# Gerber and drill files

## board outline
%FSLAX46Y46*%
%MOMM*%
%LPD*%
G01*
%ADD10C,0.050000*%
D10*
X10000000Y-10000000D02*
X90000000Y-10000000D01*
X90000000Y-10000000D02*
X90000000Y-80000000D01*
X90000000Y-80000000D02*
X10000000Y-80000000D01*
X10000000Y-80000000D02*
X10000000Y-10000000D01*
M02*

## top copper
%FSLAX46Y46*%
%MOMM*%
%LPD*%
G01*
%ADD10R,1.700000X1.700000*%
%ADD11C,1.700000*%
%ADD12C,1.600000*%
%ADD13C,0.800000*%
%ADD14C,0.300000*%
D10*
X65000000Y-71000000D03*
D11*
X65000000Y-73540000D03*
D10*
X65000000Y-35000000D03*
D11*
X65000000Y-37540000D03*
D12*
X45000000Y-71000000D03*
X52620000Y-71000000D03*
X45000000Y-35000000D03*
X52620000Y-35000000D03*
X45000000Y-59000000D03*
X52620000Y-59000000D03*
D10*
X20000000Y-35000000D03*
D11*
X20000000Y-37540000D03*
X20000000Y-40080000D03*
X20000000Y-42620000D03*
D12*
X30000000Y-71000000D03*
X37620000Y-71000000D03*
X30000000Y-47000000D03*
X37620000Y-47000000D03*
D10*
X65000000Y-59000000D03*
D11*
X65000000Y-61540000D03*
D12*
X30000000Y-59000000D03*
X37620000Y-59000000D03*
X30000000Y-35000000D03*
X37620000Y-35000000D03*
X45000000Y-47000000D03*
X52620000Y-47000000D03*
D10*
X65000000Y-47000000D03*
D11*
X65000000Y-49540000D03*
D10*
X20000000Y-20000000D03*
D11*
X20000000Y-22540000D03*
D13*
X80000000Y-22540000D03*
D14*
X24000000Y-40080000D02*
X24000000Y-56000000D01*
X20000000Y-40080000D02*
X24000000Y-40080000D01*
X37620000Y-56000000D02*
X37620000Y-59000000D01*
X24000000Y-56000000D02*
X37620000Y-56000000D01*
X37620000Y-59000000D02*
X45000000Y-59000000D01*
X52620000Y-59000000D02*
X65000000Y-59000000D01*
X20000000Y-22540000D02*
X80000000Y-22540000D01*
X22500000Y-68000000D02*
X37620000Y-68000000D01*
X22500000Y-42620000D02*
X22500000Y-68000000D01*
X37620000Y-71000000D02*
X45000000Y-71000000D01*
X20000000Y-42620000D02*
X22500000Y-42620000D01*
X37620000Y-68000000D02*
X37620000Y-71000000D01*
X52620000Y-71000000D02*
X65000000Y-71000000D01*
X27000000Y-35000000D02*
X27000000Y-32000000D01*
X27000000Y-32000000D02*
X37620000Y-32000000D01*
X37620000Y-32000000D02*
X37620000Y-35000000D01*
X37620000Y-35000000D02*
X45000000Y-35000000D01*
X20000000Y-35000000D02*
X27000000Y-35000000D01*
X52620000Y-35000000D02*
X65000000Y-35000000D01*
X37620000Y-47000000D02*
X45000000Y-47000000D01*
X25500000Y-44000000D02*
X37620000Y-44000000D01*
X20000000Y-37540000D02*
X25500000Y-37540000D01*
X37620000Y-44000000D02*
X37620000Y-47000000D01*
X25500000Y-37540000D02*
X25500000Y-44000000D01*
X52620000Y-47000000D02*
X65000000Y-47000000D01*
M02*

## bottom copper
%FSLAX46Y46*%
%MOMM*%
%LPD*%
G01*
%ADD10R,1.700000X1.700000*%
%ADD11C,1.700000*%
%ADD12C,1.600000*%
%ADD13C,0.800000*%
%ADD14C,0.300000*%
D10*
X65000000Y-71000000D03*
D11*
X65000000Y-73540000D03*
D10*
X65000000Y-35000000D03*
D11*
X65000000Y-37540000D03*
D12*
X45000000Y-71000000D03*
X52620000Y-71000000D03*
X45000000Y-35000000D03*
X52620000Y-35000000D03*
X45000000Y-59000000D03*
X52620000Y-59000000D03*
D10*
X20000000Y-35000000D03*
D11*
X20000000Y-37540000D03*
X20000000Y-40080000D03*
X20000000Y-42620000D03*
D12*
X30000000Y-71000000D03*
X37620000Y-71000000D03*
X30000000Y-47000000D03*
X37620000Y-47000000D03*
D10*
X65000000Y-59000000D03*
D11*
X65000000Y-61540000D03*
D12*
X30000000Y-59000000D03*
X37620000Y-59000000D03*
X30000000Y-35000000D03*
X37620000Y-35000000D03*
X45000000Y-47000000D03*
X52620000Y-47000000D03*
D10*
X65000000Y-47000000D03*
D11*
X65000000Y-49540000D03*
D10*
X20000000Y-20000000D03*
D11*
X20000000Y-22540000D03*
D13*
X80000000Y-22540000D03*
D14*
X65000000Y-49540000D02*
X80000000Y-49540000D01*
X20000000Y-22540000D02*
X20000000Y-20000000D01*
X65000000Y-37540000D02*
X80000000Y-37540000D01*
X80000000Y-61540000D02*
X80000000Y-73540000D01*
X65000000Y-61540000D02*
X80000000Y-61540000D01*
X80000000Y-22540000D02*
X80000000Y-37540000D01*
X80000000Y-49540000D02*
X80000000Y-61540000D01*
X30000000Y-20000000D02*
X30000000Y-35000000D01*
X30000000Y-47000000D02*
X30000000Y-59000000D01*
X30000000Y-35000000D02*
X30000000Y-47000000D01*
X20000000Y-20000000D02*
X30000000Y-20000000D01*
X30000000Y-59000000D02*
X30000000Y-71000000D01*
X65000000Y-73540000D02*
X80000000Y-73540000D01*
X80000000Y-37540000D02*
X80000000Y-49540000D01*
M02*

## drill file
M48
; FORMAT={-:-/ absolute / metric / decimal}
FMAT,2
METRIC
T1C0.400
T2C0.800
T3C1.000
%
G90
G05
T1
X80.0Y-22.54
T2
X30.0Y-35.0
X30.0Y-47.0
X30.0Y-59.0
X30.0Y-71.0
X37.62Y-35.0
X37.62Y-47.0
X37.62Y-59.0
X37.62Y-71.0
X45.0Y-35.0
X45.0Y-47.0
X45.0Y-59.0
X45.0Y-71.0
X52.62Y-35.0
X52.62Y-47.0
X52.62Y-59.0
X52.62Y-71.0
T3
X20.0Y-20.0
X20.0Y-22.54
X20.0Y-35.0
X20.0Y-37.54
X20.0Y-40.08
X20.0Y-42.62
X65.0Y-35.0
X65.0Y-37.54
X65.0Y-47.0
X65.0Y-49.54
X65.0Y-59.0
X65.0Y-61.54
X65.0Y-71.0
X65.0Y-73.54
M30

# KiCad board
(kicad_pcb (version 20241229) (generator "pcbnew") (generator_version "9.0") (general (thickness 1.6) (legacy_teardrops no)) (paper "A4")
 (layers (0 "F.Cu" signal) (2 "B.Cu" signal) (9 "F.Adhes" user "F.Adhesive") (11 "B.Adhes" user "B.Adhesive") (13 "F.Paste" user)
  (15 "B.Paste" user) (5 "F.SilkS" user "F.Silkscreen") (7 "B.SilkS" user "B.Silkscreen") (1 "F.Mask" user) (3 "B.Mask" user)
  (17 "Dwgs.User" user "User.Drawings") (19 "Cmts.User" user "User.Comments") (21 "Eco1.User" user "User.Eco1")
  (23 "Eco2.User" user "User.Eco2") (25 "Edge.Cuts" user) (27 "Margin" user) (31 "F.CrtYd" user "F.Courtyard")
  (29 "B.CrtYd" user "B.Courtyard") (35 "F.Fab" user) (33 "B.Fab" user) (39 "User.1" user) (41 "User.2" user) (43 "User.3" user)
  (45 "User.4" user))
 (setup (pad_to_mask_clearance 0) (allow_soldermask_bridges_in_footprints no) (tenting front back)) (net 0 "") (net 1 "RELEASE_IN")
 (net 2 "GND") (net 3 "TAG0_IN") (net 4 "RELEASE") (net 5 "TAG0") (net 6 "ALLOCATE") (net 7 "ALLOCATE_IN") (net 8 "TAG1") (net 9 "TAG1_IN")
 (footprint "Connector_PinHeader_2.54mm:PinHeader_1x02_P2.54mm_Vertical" (layer "F.Cu") (at 65 71)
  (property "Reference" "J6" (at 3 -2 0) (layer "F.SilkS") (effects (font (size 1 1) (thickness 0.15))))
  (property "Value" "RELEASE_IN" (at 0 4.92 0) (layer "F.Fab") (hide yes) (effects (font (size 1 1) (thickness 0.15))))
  (pad "1" thru_hole rect (at 0 0) (size 1.7 1.7) (drill 1) (layers "*.Cu" "*.Mask") (remove_unused_layers no) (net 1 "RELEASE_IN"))
  (pad "2" thru_hole circle (at 0 2.54) (size 1.7 1.7) (drill 1) (layers "*.Cu" "*.Mask") (remove_unused_layers no) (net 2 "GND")))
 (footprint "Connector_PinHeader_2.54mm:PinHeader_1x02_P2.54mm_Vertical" (layer "F.Cu") (at 65 35)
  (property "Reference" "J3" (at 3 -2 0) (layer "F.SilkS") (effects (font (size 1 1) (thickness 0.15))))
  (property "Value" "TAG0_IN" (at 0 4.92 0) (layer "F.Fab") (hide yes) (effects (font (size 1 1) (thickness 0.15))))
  (pad "1" thru_hole rect (at 0 0) (size 1.7 1.7) (drill 1) (layers "*.Cu" "*.Mask") (remove_unused_layers no) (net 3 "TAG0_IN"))
  (pad "2" thru_hole circle (at 0 2.54) (size 1.7 1.7) (drill 1) (layers "*.Cu" "*.Mask") (remove_unused_layers no) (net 2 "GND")))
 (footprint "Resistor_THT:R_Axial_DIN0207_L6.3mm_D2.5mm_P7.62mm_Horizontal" (layer "F.Cu") (at 45 71)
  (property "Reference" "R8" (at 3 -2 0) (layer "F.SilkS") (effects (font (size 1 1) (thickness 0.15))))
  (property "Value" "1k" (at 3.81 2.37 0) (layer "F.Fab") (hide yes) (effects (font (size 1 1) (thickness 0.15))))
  (pad "1" thru_hole circle (at 0 0) (size 1.6 1.6) (drill 0.8) (layers "*.Cu" "*.Mask") (remove_unused_layers no) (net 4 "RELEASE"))
  (pad "2" thru_hole circle (at 7.62 0) (size 1.6 1.6) (drill 0.8) (layers "*.Cu" "*.Mask") (remove_unused_layers no) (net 1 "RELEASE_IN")))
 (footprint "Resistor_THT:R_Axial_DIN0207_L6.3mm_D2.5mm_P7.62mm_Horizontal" (layer "F.Cu") (at 45 35)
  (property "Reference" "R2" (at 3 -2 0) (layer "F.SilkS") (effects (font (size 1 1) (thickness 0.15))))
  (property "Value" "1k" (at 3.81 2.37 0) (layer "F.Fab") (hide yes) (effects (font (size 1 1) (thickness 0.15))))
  (pad "1" thru_hole circle (at 0 0) (size 1.6 1.6) (drill 0.8) (layers "*.Cu" "*.Mask") (remove_unused_layers no) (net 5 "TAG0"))
  (pad "2" thru_hole circle (at 7.62 0) (size 1.6 1.6) (drill 0.8) (layers "*.Cu" "*.Mask") (remove_unused_layers no) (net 3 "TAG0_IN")))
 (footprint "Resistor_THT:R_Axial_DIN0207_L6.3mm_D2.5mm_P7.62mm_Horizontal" (layer "F.Cu") (at 45 59)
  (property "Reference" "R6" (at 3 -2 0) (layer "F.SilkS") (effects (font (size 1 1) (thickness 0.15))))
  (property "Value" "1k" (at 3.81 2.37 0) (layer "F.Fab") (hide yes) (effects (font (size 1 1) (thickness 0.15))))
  (pad "1" thru_hole circle (at 0 0) (size 1.6 1.6) (drill 0.8) (layers "*.Cu" "*.Mask") (remove_unused_layers no) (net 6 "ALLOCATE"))
  (pad "2" thru_hole circle (at 7.62 0) (size 1.6 1.6) (drill 0.8) (layers "*.Cu" "*.Mask") (remove_unused_layers no) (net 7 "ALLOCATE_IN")))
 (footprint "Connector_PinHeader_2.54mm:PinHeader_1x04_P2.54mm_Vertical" (layer "F.Cu") (at 20 35)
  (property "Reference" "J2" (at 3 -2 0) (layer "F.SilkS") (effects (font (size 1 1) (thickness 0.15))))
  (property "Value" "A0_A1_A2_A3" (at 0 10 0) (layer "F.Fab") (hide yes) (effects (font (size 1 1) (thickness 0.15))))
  (pad "1" thru_hole rect (at 0 0) (size 1.7 1.7) (drill 1) (layers "*.Cu" "*.Mask") (remove_unused_layers no) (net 5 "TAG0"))
  (pad "2" thru_hole circle (at 0 2.54) (size 1.7 1.7) (drill 1) (layers "*.Cu" "*.Mask") (remove_unused_layers no) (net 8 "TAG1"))
  (pad "3" thru_hole circle (at 0 5.08) (size 1.7 1.7) (drill 1) (layers "*.Cu" "*.Mask") (remove_unused_layers no) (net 6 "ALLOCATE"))
  (pad "4" thru_hole circle (at 0 7.62) (size 1.7 1.7) (drill 1) (layers "*.Cu" "*.Mask") (remove_unused_layers no) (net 4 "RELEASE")))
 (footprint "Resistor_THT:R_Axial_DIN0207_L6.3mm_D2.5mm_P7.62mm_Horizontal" (layer "F.Cu") (at 30 71)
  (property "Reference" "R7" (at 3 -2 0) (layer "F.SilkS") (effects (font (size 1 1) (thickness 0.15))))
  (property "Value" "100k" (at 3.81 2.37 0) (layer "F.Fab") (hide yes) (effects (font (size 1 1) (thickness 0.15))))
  (pad "1" thru_hole circle (at 0 0) (size 1.6 1.6) (drill 0.8) (layers "*.Cu" "*.Mask") (remove_unused_layers no) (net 2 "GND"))
  (pad "2" thru_hole circle (at 7.62 0) (size 1.6 1.6) (drill 0.8) (layers "*.Cu" "*.Mask") (remove_unused_layers no) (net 4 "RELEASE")))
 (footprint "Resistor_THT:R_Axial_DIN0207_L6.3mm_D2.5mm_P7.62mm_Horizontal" (layer "F.Cu") (at 30 47)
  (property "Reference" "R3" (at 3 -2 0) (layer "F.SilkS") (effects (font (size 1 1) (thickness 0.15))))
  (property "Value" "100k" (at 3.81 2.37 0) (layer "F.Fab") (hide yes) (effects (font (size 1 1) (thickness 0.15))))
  (pad "1" thru_hole circle (at 0 0) (size 1.6 1.6) (drill 0.8) (layers "*.Cu" "*.Mask") (remove_unused_layers no) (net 2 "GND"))
  (pad "2" thru_hole circle (at 7.62 0) (size 1.6 1.6) (drill 0.8) (layers "*.Cu" "*.Mask") (remove_unused_layers no) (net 8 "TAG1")))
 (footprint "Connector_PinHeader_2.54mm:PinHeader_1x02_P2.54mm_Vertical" (layer "F.Cu") (at 65 59)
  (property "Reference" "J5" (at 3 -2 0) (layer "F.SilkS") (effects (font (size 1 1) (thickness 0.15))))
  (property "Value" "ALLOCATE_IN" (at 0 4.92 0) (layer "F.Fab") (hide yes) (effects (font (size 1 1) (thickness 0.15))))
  (pad "1" thru_hole rect (at 0 0) (size 1.7 1.7) (drill 1) (layers "*.Cu" "*.Mask") (remove_unused_layers no) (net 7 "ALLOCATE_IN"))
  (pad "2" thru_hole circle (at 0 2.54) (size 1.7 1.7) (drill 1) (layers "*.Cu" "*.Mask") (remove_unused_layers no) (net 2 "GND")))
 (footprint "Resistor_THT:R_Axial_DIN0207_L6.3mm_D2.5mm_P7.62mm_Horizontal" (layer "F.Cu") (at 30 59)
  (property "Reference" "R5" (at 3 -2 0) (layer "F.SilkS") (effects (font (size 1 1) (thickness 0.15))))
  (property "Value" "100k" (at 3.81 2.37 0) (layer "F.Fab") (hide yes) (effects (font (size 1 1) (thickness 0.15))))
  (pad "1" thru_hole circle (at 0 0) (size 1.6 1.6) (drill 0.8) (layers "*.Cu" "*.Mask") (remove_unused_layers no) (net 2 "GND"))
  (pad "2" thru_hole circle (at 7.62 0) (size 1.6 1.6) (drill 0.8) (layers "*.Cu" "*.Mask") (remove_unused_layers no) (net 6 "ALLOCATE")))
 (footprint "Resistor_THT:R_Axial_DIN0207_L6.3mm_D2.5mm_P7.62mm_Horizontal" (layer "F.Cu") (at 30 35)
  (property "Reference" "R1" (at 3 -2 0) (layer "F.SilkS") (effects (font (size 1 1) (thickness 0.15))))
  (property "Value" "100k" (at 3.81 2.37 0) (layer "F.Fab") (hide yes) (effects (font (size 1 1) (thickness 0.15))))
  (pad "1" thru_hole circle (at 0 0) (size 1.6 1.6) (drill 0.8) (layers "*.Cu" "*.Mask") (remove_unused_layers no) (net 2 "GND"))
  (pad "2" thru_hole circle (at 7.62 0) (size 1.6 1.6) (drill 0.8) (layers "*.Cu" "*.Mask") (remove_unused_layers no) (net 5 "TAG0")))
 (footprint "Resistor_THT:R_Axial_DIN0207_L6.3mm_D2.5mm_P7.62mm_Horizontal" (layer "F.Cu") (at 45 47)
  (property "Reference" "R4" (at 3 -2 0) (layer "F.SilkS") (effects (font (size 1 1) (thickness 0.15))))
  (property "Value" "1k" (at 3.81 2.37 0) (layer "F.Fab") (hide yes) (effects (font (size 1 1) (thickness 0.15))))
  (pad "1" thru_hole circle (at 0 0) (size 1.6 1.6) (drill 0.8) (layers "*.Cu" "*.Mask") (remove_unused_layers no) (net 8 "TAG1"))
  (pad "2" thru_hole circle (at 7.62 0) (size 1.6 1.6) (drill 0.8) (layers "*.Cu" "*.Mask") (remove_unused_layers no) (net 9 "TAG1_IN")))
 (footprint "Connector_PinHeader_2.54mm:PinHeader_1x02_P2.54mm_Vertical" (layer "F.Cu") (at 65 47)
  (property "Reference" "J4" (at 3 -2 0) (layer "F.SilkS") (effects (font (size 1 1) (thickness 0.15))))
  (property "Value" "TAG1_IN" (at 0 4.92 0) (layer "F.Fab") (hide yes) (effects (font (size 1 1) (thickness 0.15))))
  (pad "1" thru_hole rect (at 0 0) (size 1.7 1.7) (drill 1) (layers "*.Cu" "*.Mask") (remove_unused_layers no) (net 9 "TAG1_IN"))
  (pad "2" thru_hole circle (at 0 2.54) (size 1.7 1.7) (drill 1) (layers "*.Cu" "*.Mask") (remove_unused_layers no) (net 2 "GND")))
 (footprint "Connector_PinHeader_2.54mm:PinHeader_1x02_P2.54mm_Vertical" (layer "F.Cu") (at 20 20)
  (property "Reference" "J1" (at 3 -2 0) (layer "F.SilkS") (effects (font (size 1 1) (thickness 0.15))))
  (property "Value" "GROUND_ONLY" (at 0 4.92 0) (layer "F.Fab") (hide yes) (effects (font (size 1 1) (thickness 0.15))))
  (pad "1" thru_hole rect (at 0 0) (size 1.7 1.7) (drill 1) (layers "*.Cu" "*.Mask") (remove_unused_layers no) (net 2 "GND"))
  (pad "2" thru_hole circle (at 0 2.54) (size 1.7 1.7) (drill 1) (layers "*.Cu" "*.Mask") (remove_unused_layers no) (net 2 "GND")))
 (gr_line (start 10 10) (end 90 10) (stroke (width 0.05) (type default)) (layer "Edge.Cuts"))
 (gr_line (start 90 10) (end 90 80) (stroke (width 0.05) (type default)) (layer "Edge.Cuts"))
 (gr_line (start 90 80) (end 10 80) (stroke (width 0.05) (type default)) (layer "Edge.Cuts"))
 (gr_line (start 10 80) (end 10 10) (stroke (width 0.05) (type default)) (layer "Edge.Cuts"))
 (segment (start 24 40.08) (end 24 56) (width 0.3) (layer "F.Cu") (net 6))
 (segment (start 20 40.08) (end 24 40.08) (width 0.3) (layer "F.Cu") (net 6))
 (segment (start 37.62 56) (end 37.62 59) (width 0.3) (layer "F.Cu") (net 6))
 (segment (start 24 56) (end 37.62 56) (width 0.3) (layer "F.Cu") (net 6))
 (segment (start 37.62 59) (end 45 59) (width 0.3) (layer "F.Cu") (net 6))
 (segment (start 52.62 59) (end 65 59) (width 0.3) (layer "F.Cu") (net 7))
 (segment (start 20 22.54) (end 80 22.54) (width 0.3) (layer "F.Cu") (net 2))
 (via (at 80 22.54) (size 0.8) (drill 0.4) (layers "F.Cu" "B.Cu") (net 2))
 (segment (start 65 49.54) (end 80 49.54) (width 0.3) (layer "B.Cu") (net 2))
 (segment (start 20 22.54) (end 20 20) (width 0.3) (layer "B.Cu") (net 2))
 (segment (start 65 37.54) (end 80 37.54) (width 0.3) (layer "B.Cu") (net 2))
 (segment (start 80 61.54) (end 80 73.54) (width 0.3) (layer "B.Cu") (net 2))
 (segment (start 65 61.54) (end 80 61.54) (width 0.3) (layer "B.Cu") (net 2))
 (segment (start 80 22.54) (end 80 37.54) (width 0.3) (layer "B.Cu") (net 2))
 (segment (start 80 49.54) (end 80 61.54) (width 0.3) (layer "B.Cu") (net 2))
 (segment (start 30 20) (end 30 35) (width 0.3) (layer "B.Cu") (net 2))
 (segment (start 30 47) (end 30 59) (width 0.3) (layer "B.Cu") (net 2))
 (segment (start 30 35) (end 30 47) (width 0.3) (layer "B.Cu") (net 2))
 (segment (start 20 20) (end 30 20) (width 0.3) (layer "B.Cu") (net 2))
 (segment (start 30 59) (end 30 71) (width 0.3) (layer "B.Cu") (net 2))
 (segment (start 65 73.54) (end 80 73.54) (width 0.3) (layer "B.Cu") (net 2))
 (segment (start 80 37.54) (end 80 49.54) (width 0.3) (layer "B.Cu") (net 2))
 (segment (start 22.5 68) (end 37.62 68) (width 0.3) (layer "F.Cu") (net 4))
 (segment (start 22.5 42.62) (end 22.5 68) (width 0.3) (layer "F.Cu") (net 4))
 (segment (start 37.62 71) (end 45 71) (width 0.3) (layer "F.Cu") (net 4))
 (segment (start 20 42.62) (end 22.5 42.62) (width 0.3) (layer "F.Cu") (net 4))
 (segment (start 37.62 68) (end 37.62 71) (width 0.3) (layer "F.Cu") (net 4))
 (segment (start 52.62 71) (end 65 71) (width 0.3) (layer "F.Cu") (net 1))
 (segment (start 27 35) (end 27 32) (width 0.3) (layer "F.Cu") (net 5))
 (segment (start 27 32) (end 37.62 32) (width 0.3) (layer "F.Cu") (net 5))
 (segment (start 37.62 32) (end 37.62 35) (width 0.3) (layer "F.Cu") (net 5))
 (segment (start 37.62 35) (end 45 35) (width 0.3) (layer "F.Cu") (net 5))
 (segment (start 20 35) (end 27 35) (width 0.3) (layer "F.Cu") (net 5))
 (segment (start 52.62 35) (end 65 35) (width 0.3) (layer "F.Cu") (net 3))
 (segment (start 37.62 47) (end 45 47) (width 0.3) (layer "F.Cu") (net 8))
 (segment (start 25.5 44) (end 37.62 44) (width 0.3) (layer "F.Cu") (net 8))
 (segment (start 20 37.54) (end 25.5 37.54) (width 0.3) (layer "F.Cu") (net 8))
 (segment (start 37.62 44) (end 37.62 47) (width 0.3) (layer "F.Cu") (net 8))
 (segment (start 25.5 37.54) (end 25.5 44) (width 0.3) (layer "F.Cu") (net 8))
 (segment (start 52.62 47) (end 65 47) (width 0.3) (layer "F.Cu") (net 9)))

